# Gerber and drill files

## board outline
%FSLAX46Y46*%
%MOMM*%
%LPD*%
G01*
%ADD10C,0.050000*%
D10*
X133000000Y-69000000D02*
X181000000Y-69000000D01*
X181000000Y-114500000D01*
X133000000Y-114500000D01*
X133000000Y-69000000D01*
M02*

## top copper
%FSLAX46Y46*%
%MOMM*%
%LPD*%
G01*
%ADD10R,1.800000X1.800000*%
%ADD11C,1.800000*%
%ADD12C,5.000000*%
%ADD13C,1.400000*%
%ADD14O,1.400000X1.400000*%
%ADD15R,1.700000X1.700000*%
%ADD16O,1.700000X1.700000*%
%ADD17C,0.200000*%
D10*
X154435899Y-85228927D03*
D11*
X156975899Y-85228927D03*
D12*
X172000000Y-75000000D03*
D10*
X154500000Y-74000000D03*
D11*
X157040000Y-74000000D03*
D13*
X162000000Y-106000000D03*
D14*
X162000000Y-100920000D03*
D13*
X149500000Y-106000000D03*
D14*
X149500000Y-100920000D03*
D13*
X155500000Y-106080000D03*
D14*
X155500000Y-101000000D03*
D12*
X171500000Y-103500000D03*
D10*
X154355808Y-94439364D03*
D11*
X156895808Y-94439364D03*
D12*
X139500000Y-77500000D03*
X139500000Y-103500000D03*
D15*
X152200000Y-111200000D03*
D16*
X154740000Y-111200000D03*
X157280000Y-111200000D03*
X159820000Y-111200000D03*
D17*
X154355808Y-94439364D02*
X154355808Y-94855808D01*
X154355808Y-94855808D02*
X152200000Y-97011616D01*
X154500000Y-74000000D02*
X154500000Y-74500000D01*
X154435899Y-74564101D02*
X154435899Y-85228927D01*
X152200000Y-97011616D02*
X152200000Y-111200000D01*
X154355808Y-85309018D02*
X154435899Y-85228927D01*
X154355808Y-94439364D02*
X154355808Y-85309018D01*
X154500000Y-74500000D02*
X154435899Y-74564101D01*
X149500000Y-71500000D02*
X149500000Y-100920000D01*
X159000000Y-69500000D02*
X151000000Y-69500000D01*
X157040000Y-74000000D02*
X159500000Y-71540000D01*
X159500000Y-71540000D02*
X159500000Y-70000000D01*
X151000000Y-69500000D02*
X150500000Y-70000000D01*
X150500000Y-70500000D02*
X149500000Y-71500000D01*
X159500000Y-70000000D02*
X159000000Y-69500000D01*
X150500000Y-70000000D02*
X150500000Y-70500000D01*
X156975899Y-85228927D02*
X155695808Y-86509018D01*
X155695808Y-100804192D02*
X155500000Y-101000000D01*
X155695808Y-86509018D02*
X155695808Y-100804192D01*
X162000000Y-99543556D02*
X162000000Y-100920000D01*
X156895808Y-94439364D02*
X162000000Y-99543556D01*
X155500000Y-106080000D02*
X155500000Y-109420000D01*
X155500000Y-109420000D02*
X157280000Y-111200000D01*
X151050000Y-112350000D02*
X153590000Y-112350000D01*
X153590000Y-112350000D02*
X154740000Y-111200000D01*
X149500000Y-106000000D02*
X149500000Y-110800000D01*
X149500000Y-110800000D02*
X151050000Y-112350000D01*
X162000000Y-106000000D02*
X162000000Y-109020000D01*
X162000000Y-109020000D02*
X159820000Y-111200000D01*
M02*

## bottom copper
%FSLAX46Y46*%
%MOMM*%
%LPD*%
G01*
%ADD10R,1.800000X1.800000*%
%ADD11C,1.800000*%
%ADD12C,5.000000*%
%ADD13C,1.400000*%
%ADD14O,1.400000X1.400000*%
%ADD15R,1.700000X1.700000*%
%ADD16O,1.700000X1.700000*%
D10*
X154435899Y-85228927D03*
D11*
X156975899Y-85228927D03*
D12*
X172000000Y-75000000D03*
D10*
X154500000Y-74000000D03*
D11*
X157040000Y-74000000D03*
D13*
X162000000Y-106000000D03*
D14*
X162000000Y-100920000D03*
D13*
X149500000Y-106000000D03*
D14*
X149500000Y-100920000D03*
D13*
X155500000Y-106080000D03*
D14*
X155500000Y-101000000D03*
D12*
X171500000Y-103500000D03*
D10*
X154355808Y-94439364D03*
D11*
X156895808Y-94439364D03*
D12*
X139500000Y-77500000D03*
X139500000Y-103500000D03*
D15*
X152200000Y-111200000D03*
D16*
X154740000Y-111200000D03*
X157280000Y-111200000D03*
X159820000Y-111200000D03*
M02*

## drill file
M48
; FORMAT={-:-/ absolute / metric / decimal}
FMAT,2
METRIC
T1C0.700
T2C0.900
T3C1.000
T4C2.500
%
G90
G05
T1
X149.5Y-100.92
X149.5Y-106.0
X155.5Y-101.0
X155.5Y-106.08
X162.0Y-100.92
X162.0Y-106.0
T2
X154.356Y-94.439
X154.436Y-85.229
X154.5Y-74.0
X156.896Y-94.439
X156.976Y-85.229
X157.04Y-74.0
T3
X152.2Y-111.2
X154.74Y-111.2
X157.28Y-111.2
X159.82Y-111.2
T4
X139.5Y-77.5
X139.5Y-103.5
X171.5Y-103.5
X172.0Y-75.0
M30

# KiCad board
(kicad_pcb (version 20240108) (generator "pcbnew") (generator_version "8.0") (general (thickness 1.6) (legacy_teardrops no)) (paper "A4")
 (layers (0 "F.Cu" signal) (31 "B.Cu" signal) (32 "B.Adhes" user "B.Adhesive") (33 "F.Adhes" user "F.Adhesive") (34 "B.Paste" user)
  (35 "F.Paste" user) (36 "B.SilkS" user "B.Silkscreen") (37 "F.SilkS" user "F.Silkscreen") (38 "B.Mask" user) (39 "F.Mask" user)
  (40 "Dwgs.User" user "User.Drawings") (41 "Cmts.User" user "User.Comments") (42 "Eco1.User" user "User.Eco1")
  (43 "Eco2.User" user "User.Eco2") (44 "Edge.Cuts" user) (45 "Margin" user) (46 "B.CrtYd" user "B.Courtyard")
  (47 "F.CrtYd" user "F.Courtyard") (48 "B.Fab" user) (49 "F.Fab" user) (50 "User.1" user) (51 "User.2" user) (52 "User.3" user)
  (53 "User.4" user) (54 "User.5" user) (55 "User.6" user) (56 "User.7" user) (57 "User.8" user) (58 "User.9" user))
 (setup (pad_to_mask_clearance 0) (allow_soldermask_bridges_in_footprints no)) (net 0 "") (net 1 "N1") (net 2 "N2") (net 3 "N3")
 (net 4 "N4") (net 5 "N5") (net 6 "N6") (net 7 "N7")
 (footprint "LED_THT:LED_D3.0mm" (layer "F.Cu") (at 154.435899 85.228927)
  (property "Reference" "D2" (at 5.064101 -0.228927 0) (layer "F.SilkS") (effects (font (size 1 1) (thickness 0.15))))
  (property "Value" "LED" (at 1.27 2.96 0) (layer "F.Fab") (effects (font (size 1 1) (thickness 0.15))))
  (pad "1" thru_hole rect (at 0 0) (size 1.8 1.8) (drill 0.9) (layers "*.Cu" "*.Mask") (remove_unused_layers no) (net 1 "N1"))
  (pad "2" thru_hole circle (at 2.54 0) (size 1.8 1.8) (drill 0.9) (layers "*.Cu" "*.Mask") (remove_unused_layers no) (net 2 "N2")))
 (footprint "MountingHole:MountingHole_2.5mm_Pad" (layer "F.Cu") (at 172 75)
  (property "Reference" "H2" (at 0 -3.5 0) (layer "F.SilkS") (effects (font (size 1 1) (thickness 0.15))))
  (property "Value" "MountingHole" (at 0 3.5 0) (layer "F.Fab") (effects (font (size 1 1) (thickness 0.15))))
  (pad "1" thru_hole circle (at 0 0) (size 5 5) (drill 2.5) (layers "*.Cu" "*.Mask") (remove_unused_layers no)))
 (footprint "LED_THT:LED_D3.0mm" (layer "F.Cu") (at 154.5 74)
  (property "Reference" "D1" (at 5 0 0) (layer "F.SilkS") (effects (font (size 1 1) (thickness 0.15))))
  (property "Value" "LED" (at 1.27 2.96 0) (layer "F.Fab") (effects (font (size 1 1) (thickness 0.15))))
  (pad "1" thru_hole rect (at 0 0) (size 1.8 1.8) (drill 0.9) (layers "*.Cu" "*.Mask") (remove_unused_layers no) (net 1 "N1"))
  (pad "2" thru_hole circle (at 2.54 0) (size 1.8 1.8) (drill 0.9) (layers "*.Cu" "*.Mask") (remove_unused_layers no) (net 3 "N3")))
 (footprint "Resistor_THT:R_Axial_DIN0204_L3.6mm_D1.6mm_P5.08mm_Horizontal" (layer "F.Cu") (at 162 106 90)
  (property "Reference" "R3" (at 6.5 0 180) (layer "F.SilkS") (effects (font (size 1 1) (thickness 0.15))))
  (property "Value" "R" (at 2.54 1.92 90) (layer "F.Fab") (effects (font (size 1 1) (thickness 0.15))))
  (pad "1" thru_hole circle (at 0 0 90) (size 1.4 1.4) (drill 0.7) (layers "*.Cu" "*.Mask") (remove_unused_layers no) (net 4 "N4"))
  (pad "2" thru_hole oval (at 5.08 0 90) (size 1.4 1.4) (drill 0.7) (layers "*.Cu" "*.Mask") (remove_unused_layers no) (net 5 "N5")))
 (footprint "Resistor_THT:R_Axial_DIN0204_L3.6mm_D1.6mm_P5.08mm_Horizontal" (layer "F.Cu") (at 149.5 106 90)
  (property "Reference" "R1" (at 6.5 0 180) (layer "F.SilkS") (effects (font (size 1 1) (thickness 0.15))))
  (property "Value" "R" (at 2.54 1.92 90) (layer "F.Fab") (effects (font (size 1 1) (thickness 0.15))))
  (pad "1" thru_hole circle (at 0 0 90) (size 1.4 1.4) (drill 0.7) (layers "*.Cu" "*.Mask") (remove_unused_layers no) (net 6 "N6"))
  (pad "2" thru_hole oval (at 5.08 0 90) (size 1.4 1.4) (drill 0.7) (layers "*.Cu" "*.Mask") (remove_unused_layers no) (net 3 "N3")))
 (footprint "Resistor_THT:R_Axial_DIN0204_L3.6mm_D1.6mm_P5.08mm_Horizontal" (layer "F.Cu") (at 155.5 106.08 90)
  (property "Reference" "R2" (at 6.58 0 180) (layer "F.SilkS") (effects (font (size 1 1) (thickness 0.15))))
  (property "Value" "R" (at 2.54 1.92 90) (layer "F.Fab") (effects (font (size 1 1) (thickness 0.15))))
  (pad "1" thru_hole circle (at 0 0 90) (size 1.4 1.4) (drill 0.7) (layers "*.Cu" "*.Mask") (remove_unused_layers no) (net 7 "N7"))
  (pad "2" thru_hole oval (at 5.08 0 90) (size 1.4 1.4) (drill 0.7) (layers "*.Cu" "*.Mask") (remove_unused_layers no) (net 2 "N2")))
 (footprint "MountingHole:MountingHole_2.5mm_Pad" (layer "F.Cu") (at 171.5 103.5)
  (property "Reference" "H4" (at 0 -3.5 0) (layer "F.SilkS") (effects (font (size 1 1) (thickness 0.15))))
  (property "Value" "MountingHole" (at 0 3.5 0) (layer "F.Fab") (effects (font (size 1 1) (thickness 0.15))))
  (pad "1" thru_hole circle (at 0 0) (size 5 5) (drill 2.5) (layers "*.Cu" "*.Mask") (remove_unused_layers no)))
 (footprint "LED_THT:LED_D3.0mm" (layer "F.Cu") (at 154.355808 94.439364)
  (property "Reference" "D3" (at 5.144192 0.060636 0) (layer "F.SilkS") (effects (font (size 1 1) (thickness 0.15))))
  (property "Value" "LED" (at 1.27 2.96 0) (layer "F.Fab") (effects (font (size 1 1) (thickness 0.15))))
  (pad "1" thru_hole rect (at 0 0) (size 1.8 1.8) (drill 0.9) (layers "*.Cu" "*.Mask") (remove_unused_layers no) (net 1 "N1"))
  (pad "2" thru_hole circle (at 2.54 0) (size 1.8 1.8) (drill 0.9) (layers "*.Cu" "*.Mask") (remove_unused_layers no) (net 5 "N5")))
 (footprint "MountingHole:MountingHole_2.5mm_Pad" (layer "F.Cu") (at 139.5 77.5)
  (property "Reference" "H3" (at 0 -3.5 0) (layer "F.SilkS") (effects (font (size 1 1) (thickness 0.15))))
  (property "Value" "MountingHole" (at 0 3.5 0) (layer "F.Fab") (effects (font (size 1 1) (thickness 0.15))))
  (pad "1" thru_hole circle (at 0 0) (size 5 5) (drill 2.5) (layers "*.Cu" "*.Mask") (remove_unused_layers no)))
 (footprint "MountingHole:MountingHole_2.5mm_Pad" (layer "F.Cu") (at 139.5 103.5)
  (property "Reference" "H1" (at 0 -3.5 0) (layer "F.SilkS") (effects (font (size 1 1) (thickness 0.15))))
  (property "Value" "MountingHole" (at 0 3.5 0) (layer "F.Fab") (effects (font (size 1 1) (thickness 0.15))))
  (pad "1" thru_hole circle (at 0 0) (size 5 5) (drill 2.5) (layers "*.Cu" "*.Mask") (remove_unused_layers no)))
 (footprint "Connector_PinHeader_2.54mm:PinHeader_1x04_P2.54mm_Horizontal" (layer "B.Cu") (at 152.2 111.2 -90)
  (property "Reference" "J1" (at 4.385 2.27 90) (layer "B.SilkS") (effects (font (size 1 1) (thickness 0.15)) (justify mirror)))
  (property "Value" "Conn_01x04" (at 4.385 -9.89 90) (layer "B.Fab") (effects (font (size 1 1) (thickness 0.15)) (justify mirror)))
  (pad "1" thru_hole rect (at 0 0 270) (size 1.7 1.7) (drill 1) (layers "*.Cu" "*.Mask") (remove_unused_layers no) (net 1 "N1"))
  (pad "2" thru_hole oval (at 0 -2.54 270) (size 1.7 1.7) (drill 1) (layers "*.Cu" "*.Mask") (remove_unused_layers no) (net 6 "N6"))
  (pad "3" thru_hole oval (at 0 -5.08 270) (size 1.7 1.7) (drill 1) (layers "*.Cu" "*.Mask") (remove_unused_layers no) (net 7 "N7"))
  (pad "4" thru_hole oval (at 0 -7.62 270) (size 1.7 1.7) (drill 1) (layers "*.Cu" "*.Mask") (remove_unused_layers no) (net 4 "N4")))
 (gr_rect (start 133 69) (end 181 114.5) (stroke (width 0.05) (type default)) (fill none) (layer "Edge.Cuts"))
 (segment (start 154.355808 94.439364) (end 154.355808 94.855808) (width 0.2) (layer "F.Cu") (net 1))
 (segment (start 154.355808 94.855808) (end 152.2 97.011616) (width 0.2) (layer "F.Cu") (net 1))
 (segment (start 154.5 74) (end 154.5 74.5) (width 0.2) (layer "F.Cu") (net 1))
 (segment (start 154.435899 74.564101) (end 154.435899 85.228927) (width 0.2) (layer "F.Cu") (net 1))
 (segment (start 152.2 97.011616) (end 152.2 111.2) (width 0.2) (layer "F.Cu") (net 1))
 (segment (start 154.355808 85.309018) (end 154.435899 85.228927) (width 0.2) (layer "F.Cu") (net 1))
 (segment (start 154.355808 94.439364) (end 154.355808 85.309018) (width 0.2) (layer "F.Cu") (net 1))
 (segment (start 154.5 74.5) (end 154.435899 74.564101) (width 0.2) (layer "F.Cu") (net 1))
 (segment (start 149.5 71.5) (end 149.5 100.92) (width 0.2) (layer "F.Cu") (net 3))
 (segment (start 159 69.5) (end 151 69.5) (width 0.2) (layer "F.Cu") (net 3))
 (segment (start 157.04 74) (end 159.5 71.54) (width 0.2) (layer "F.Cu") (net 3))
 (segment (start 159.5 71.54) (end 159.5 70) (width 0.2) (layer "F.Cu") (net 3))
 (segment (start 151 69.5) (end 150.5 70) (width 0.2) (layer "F.Cu") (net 3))
 (segment (start 150.5 70.5) (end 149.5 71.5) (width 0.2) (layer "F.Cu") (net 3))
 (segment (start 159.5 70) (end 159 69.5) (width 0.2) (layer "F.Cu") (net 3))
 (segment (start 150.5 70) (end 150.5 70.5) (width 0.2) (layer "F.Cu") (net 3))
 (segment (start 156.975899 85.228927) (end 155.695808 86.509018) (width 0.2) (layer "F.Cu") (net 2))
 (segment (start 155.695808 100.804192) (end 155.5 101) (width 0.2) (layer "F.Cu") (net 2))
 (segment (start 155.695808 86.509018) (end 155.695808 100.804192) (width 0.2) (layer "F.Cu") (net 2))
 (segment (start 162 99.543556) (end 162 100.92) (width 0.2) (layer "F.Cu") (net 5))
 (segment (start 156.895808 94.439364) (end 162 99.543556) (width 0.2) (layer "F.Cu") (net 5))
 (segment (start 155.5 106.08) (end 155.5 109.42) (width 0.2) (layer "F.Cu") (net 7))
 (segment (start 155.5 109.42) (end 157.28 111.2) (width 0.2) (layer "F.Cu") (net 7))
 (segment (start 151.05 112.35) (end 153.59 112.35) (width 0.2) (layer "F.Cu") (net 6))
 (segment (start 153.59 112.35) (end 154.74 111.2) (width 0.2) (layer "F.Cu") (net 6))
 (segment (start 149.5 106) (end 149.5 110.8) (width 0.2) (layer "F.Cu") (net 6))
 (segment (start 149.5 110.8) (end 151.05 112.35) (width 0.2) (layer "F.Cu") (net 6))
 (segment (start 162 106) (end 162 109.02) (width 0.2) (layer "F.Cu") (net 4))
 (segment (start 162 109.02) (end 159.82 111.2) (width 0.2) (layer "F.Cu") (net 4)))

